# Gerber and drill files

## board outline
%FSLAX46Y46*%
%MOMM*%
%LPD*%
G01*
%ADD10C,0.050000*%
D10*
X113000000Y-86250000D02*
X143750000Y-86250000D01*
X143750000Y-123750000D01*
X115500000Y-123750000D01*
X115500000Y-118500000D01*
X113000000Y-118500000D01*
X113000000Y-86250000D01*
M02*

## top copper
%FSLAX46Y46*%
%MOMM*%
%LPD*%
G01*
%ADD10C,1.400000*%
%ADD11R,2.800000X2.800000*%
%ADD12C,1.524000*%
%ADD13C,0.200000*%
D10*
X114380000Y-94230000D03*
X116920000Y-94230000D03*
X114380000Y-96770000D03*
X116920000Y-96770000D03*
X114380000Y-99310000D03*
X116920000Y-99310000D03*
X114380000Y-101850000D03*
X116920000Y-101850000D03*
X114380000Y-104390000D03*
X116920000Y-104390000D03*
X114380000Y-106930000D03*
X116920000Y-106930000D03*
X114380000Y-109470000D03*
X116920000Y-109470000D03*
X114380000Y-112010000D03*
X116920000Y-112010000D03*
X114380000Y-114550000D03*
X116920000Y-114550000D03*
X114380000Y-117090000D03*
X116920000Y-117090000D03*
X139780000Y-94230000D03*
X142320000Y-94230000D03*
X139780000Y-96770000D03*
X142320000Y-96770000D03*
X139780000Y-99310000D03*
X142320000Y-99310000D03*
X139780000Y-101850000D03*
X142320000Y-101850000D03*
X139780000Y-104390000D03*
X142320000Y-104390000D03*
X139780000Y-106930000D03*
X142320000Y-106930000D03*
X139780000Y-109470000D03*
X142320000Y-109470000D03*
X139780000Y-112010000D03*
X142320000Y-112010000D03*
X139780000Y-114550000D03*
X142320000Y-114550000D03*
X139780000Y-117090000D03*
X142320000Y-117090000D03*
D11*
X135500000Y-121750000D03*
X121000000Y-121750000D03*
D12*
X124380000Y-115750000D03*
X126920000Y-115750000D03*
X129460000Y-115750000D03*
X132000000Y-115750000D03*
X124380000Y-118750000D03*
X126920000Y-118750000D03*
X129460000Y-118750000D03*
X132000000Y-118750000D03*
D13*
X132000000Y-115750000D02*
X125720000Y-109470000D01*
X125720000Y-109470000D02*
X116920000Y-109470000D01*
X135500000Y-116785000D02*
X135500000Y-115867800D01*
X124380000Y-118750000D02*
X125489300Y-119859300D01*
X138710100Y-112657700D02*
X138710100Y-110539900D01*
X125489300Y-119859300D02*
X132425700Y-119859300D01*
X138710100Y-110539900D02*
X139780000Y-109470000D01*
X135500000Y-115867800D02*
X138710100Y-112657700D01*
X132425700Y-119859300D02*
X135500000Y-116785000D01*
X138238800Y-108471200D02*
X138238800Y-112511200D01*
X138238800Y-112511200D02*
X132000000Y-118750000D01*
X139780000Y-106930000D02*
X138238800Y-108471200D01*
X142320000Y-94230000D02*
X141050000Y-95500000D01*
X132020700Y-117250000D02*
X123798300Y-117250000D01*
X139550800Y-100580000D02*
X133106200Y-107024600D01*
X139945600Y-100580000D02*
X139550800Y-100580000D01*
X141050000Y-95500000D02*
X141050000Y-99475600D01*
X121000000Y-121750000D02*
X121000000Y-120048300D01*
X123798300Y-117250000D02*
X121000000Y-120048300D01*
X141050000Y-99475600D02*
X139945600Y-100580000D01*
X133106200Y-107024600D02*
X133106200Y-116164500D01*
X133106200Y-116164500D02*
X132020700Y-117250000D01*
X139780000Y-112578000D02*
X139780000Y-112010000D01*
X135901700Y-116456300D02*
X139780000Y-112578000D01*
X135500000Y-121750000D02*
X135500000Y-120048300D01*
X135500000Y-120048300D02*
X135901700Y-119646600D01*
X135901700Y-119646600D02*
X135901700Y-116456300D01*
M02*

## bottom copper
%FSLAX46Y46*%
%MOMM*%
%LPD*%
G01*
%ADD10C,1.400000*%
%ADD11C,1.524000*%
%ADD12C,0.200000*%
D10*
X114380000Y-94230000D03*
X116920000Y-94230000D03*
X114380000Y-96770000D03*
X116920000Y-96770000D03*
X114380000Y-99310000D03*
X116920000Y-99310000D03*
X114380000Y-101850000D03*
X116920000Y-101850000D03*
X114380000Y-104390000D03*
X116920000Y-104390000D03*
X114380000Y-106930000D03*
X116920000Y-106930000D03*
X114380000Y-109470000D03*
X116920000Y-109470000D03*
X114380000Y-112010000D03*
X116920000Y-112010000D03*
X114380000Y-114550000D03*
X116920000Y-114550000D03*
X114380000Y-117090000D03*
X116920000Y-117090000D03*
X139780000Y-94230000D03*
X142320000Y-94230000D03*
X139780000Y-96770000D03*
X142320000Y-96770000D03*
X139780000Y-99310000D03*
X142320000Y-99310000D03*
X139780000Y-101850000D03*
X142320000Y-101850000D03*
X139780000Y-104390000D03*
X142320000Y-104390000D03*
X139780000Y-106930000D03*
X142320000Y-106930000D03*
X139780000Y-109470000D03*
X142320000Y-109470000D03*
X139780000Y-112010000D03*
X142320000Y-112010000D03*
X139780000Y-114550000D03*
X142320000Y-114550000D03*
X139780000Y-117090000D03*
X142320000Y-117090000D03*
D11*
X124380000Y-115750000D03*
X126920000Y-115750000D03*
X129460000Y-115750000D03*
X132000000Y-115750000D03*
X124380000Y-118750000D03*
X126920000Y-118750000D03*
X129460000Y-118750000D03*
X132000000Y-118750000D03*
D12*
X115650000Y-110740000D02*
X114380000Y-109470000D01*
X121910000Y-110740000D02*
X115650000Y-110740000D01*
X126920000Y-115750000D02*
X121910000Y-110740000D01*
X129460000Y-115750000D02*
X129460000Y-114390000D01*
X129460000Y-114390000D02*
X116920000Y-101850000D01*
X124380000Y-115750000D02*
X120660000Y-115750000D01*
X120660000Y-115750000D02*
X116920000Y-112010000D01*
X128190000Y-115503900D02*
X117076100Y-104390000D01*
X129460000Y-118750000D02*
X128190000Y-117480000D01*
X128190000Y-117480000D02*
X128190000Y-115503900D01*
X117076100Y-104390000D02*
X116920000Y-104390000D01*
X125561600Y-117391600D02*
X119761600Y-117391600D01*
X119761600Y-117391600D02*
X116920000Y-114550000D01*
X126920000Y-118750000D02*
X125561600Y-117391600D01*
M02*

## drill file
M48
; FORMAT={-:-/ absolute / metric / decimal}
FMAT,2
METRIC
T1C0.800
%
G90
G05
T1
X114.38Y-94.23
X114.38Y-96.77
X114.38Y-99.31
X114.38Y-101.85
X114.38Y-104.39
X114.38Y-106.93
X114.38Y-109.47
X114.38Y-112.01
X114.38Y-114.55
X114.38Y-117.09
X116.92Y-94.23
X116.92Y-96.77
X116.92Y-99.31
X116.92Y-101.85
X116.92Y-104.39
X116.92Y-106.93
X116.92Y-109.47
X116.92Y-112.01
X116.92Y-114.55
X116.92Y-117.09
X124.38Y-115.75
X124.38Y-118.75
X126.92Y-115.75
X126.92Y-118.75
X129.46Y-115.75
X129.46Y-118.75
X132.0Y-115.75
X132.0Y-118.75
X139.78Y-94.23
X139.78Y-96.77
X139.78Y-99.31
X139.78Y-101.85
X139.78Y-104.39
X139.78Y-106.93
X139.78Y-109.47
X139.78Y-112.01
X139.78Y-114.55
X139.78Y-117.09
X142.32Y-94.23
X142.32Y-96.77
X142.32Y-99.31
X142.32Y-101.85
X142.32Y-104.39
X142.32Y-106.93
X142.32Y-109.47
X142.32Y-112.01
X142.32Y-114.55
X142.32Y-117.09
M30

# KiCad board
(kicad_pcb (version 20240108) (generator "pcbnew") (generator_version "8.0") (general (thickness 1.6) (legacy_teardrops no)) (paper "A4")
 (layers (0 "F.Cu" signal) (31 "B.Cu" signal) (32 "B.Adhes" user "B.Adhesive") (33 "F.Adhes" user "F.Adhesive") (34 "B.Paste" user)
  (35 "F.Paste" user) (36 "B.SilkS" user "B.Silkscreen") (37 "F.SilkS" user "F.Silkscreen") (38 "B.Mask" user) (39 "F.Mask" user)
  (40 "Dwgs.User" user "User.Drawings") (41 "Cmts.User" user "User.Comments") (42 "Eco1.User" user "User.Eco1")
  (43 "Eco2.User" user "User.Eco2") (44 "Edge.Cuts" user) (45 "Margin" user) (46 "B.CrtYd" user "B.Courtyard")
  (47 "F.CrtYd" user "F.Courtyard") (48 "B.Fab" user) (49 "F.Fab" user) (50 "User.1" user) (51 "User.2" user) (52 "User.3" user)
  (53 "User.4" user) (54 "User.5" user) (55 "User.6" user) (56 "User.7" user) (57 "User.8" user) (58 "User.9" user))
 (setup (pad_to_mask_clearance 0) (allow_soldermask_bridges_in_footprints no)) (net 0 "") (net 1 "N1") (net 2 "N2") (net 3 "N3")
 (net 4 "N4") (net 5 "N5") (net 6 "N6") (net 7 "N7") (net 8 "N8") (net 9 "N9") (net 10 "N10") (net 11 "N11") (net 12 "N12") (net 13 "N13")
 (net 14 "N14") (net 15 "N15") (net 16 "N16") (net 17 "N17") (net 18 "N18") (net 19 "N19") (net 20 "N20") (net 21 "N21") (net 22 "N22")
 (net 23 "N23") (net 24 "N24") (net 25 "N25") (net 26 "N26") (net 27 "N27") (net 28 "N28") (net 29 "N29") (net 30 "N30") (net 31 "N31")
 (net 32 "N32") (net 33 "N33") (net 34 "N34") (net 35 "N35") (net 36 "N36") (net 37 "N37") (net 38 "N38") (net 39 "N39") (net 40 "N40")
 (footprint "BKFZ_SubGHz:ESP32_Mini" (layer "F.Cu") (at 128.35 105.66)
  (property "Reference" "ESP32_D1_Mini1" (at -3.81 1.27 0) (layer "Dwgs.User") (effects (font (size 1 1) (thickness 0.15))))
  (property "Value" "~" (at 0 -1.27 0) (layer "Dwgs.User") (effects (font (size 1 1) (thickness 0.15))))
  (pad "1" thru_hole circle (at -13.97 -11.43 270) (size 1.4 1.4) (drill 0.8) (layers "*.Cu" "*.Mask") (remove_unused_layers no)
   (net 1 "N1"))
  (pad "2" thru_hole circle (at -11.43 -11.43 270) (size 1.4 1.4) (drill 0.8) (layers "*.Cu" "*.Mask") (remove_unused_layers no)
   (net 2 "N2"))
  (pad "3" thru_hole circle (at -13.97 -8.89 270) (size 1.4 1.4) (drill 0.8) (layers "*.Cu" "*.Mask") (remove_unused_layers no) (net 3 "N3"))
  (pad "4" thru_hole circle (at -11.43 -8.89 270) (size 1.4 1.4) (drill 0.8) (layers "*.Cu" "*.Mask") (remove_unused_layers no) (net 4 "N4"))
  (pad "5" thru_hole circle (at -13.97 -6.35 270) (size 1.4 1.4) (drill 0.8) (layers "*.Cu" "*.Mask") (remove_unused_layers no) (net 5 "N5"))
  (pad "6" thru_hole circle (at -11.43 -6.35 270) (size 1.4 1.4) (drill 0.8) (layers "*.Cu" "*.Mask") (remove_unused_layers no) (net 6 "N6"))
  (pad "7" thru_hole circle (at -13.97 -3.81 270) (size 1.4 1.4) (drill 0.8) (layers "*.Cu" "*.Mask") (remove_unused_layers no) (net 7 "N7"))
  (pad "8" thru_hole circle (at -11.43 -3.81 270) (size 1.4 1.4) (drill 0.8) (layers "*.Cu" "*.Mask") (remove_unused_layers no) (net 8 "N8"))
  (pad "9" thru_hole circle (at -13.97 -1.27 270) (size 1.4 1.4) (drill 0.8) (layers "*.Cu" "*.Mask") (remove_unused_layers no) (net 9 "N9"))
  (pad "10" thru_hole circle (at -11.43 -1.27 270) (size 1.4 1.4) (drill 0.8) (layers "*.Cu" "*.Mask") (remove_unused_layers no)
   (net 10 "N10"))
  (pad "11" thru_hole circle (at -13.97 1.27 270) (size 1.4 1.4) (drill 0.8) (layers "*.Cu" "*.Mask") (remove_unused_layers no)
   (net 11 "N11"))
  (pad "12" thru_hole circle (at -11.43 1.27 270) (size 1.4 1.4) (drill 0.8) (layers "*.Cu" "*.Mask") (remove_unused_layers no)
   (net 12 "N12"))
  (pad "13" thru_hole circle (at -13.97 3.81 270) (size 1.4 1.4) (drill 0.8) (layers "*.Cu" "*.Mask") (remove_unused_layers no)
   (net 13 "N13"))
  (pad "14" thru_hole circle (at -11.43 3.81 270) (size 1.4 1.4) (drill 0.8) (layers "*.Cu" "*.Mask") (remove_unused_layers no)
   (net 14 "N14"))
  (pad "15" thru_hole circle (at -13.97 6.35 270) (size 1.4 1.4) (drill 0.8) (layers "*.Cu" "*.Mask") (remove_unused_layers no)
   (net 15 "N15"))
  (pad "16" thru_hole circle (at -11.43 6.35 270) (size 1.4 1.4) (drill 0.8) (layers "*.Cu" "*.Mask") (remove_unused_layers no)
   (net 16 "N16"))
  (pad "17" thru_hole circle (at -13.97 8.89 270) (size 1.4 1.4) (drill 0.8) (layers "*.Cu" "*.Mask") (remove_unused_layers no)
   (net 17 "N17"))
  (pad "18" thru_hole circle (at -11.43 8.89 270) (size 1.4 1.4) (drill 0.8) (layers "*.Cu" "*.Mask") (remove_unused_layers no)
   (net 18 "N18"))
  (pad "19" thru_hole circle (at -13.97 11.43 270) (size 1.4 1.4) (drill 0.8) (layers "*.Cu" "*.Mask") (remove_unused_layers no)
   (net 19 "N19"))
  (pad "20" thru_hole circle (at -11.43 11.43 270) (size 1.4 1.4) (drill 0.8) (layers "*.Cu" "*.Mask") (remove_unused_layers no)
   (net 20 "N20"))
  (pad "21" thru_hole circle (at 11.43 -11.43 270) (size 1.4 1.4) (drill 0.8) (layers "*.Cu" "*.Mask") (remove_unused_layers no)
   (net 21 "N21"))
  (pad "22" thru_hole circle (at 13.97 -11.43 270) (size 1.4 1.4) (drill 0.8) (layers "*.Cu" "*.Mask") (remove_unused_layers no)
   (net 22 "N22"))
  (pad "23" thru_hole circle (at 11.43 -8.89 270) (size 1.4 1.4) (drill 0.8) (layers "*.Cu" "*.Mask") (remove_unused_layers no)
   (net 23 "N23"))
  (pad "24" thru_hole circle (at 13.97 -8.89 270) (size 1.4 1.4) (drill 0.8) (layers "*.Cu" "*.Mask") (remove_unused_layers no)
   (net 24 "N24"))
  (pad "25" thru_hole circle (at 11.43 -6.35 270) (size 1.4 1.4) (drill 0.8) (layers "*.Cu" "*.Mask") (remove_unused_layers no)
   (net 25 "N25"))
  (pad "26" thru_hole circle (at 13.97 -6.35 270) (size 1.4 1.4) (drill 0.8) (layers "*.Cu" "*.Mask") (remove_unused_layers no)
   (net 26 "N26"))
  (pad "27" thru_hole circle (at 11.43 -3.81 270) (size 1.4 1.4) (drill 0.8) (layers "*.Cu" "*.Mask") (remove_unused_layers no)
   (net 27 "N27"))
  (pad "28" thru_hole circle (at 13.97 -3.81 270) (size 1.4 1.4) (drill 0.8) (layers "*.Cu" "*.Mask") (remove_unused_layers no)
   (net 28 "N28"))
  (pad "29" thru_hole circle (at 11.43 -1.27 270) (size 1.4 1.4) (drill 0.8) (layers "*.Cu" "*.Mask") (remove_unused_layers no)
   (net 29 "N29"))
  (pad "30" thru_hole circle (at 13.97 -1.27 270) (size 1.4 1.4) (drill 0.8) (layers "*.Cu" "*.Mask") (remove_unused_layers no)
   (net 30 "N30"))
  (pad "31" thru_hole circle (at 11.43 1.27 270) (size 1.4 1.4) (drill 0.8) (layers "*.Cu" "*.Mask") (remove_unused_layers no)
   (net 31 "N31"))
  (pad "32" thru_hole circle (at 13.97 1.27 270) (size 1.4 1.4) (drill 0.8) (layers "*.Cu" "*.Mask") (remove_unused_layers no)
   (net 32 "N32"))
  (pad "33" thru_hole circle (at 11.43 3.81 270) (size 1.4 1.4) (drill 0.8) (layers "*.Cu" "*.Mask") (remove_unused_layers no)
   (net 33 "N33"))
  (pad "34" thru_hole circle (at 13.97 3.81 270) (size 1.4 1.4) (drill 0.8) (layers "*.Cu" "*.Mask") (remove_unused_layers no)
   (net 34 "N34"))
  (pad "35" thru_hole circle (at 11.43 6.35 270) (size 1.4 1.4) (drill 0.8) (layers "*.Cu" "*.Mask") (remove_unused_layers no)
   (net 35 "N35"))
  (pad "36" thru_hole circle (at 13.97 6.35 270) (size 1.4 1.4) (drill 0.8) (layers "*.Cu" "*.Mask") (remove_unused_layers no)
   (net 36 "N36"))
  (pad "37" thru_hole circle (at 11.43 8.89 270) (size 1.4 1.4) (drill 0.8) (layers "*.Cu" "*.Mask") (remove_unused_layers no)
   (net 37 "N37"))
  (pad "38" thru_hole circle (at 13.97 8.89 270) (size 1.4 1.4) (drill 0.8) (layers "*.Cu" "*.Mask") (remove_unused_layers no)
   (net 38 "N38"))
  (pad "39" thru_hole circle (at 11.43 11.43 270) (size 1.4 1.4) (drill 0.8) (layers "*.Cu" "*.Mask") (remove_unused_layers no)
   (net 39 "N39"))
  (pad "40" thru_hole circle (at 13.97 11.43 270) (size 1.4 1.4) (drill 0.8) (layers "*.Cu" "*.Mask") (remove_unused_layers no)
   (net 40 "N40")))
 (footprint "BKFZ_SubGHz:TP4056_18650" (layer "F.Cu") (at 137.2 97.15 -90)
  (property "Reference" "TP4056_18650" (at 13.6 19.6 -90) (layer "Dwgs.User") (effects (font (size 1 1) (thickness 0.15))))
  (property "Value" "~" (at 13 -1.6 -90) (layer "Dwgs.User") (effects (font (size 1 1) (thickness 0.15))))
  (pad "3" smd rect (at 24.6 1.7 270) (size 2.8 2.8) (layers "F.Cu" "F.Paste" "F.Mask") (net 35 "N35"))
  (pad "4" smd rect (at 24.6 16.2 270) (size 2.8 2.8) (layers "F.Cu" "F.Paste" "F.Mask") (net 22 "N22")))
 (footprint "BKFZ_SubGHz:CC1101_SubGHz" (layer "F.Cu") (at 153.685 71.9)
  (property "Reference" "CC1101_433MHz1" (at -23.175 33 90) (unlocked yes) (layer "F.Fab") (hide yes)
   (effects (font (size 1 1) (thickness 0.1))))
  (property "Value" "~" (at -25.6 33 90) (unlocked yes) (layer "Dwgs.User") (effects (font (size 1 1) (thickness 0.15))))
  (pad "1" thru_hole circle (at -29.305 43.85 270) (size 1.524 1.524) (drill 0.8) (layers "*.Cu" "*.Mask") (remove_unused_layers no)
   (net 16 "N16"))
  (pad "2" thru_hole circle (at -26.765 43.85 270) (size 1.524 1.524) (drill 0.8) (layers "*.Cu" "*.Mask") (remove_unused_layers no)
   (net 13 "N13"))
  (pad "3" thru_hole circle (at -24.225 43.85 270) (size 1.524 1.524) (drill 0.8) (layers "*.Cu" "*.Mask") (remove_unused_layers no)
   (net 8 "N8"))
  (pad "4" thru_hole circle (at -21.685 43.85 270) (size 1.524 1.524) (drill 0.8) (layers "*.Cu" "*.Mask") (remove_unused_layers no)
   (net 14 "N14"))
  (pad "5" thru_hole circle (at -29.305 46.85 270) (size 1.524 1.524) (drill 0.8) (layers "*.Cu" "*.Mask") (remove_unused_layers no)
   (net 33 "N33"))
  (pad "6" thru_hole circle (at -26.765 46.85 270) (size 1.524 1.524) (drill 0.8) (layers "*.Cu" "*.Mask") (remove_unused_layers no)
   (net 18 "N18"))
  (pad "7" thru_hole circle (at -24.225 46.85 270) (size 1.524 1.524) (drill 0.8) (layers "*.Cu" "*.Mask") (remove_unused_layers no)
   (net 10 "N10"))
  (pad "8" thru_hole circle (at -21.685 46.85 270) (size 1.524 1.524) (drill 0.8) (layers "*.Cu" "*.Mask") (remove_unused_layers no)
   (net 31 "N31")))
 (gr_poly
  (pts (xy 113 86.25) (xy 143.75 86.25) (xy 143.75 123.75) (xy 115.5 123.75) (xy 115.5 118.5) (xy 113 118.5))
  (stroke (width 0.05) (type solid)) (fill none) (layer "Edge.Cuts"))
 (segment (start 115.65 110.74) (end 114.38 109.47) (width 0.2) (layer "B.Cu") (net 13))
 (segment (start 121.91 110.74) (end 115.65 110.74) (width 0.2) (layer "B.Cu") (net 13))
 (segment (start 126.92 115.75) (end 121.91 110.74) (width 0.2) (layer "B.Cu") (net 13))
 (segment (start 129.46 115.75) (end 129.46 114.39) (width 0.2) (layer "B.Cu") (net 8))
 (segment (start 129.46 114.39) (end 116.92 101.85) (width 0.2) (layer "B.Cu") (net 8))
 (segment (start 132 115.75) (end 125.72 109.47) (width 0.2) (layer "F.Cu") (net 14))
 (segment (start 125.72 109.47) (end 116.92 109.47) (width 0.2) (layer "F.Cu") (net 14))
 (segment (start 124.38 115.75) (end 120.66 115.75) (width 0.2) (layer "B.Cu") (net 16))
 (segment (start 120.66 115.75) (end 116.92 112.01) (width 0.2) (layer "B.Cu") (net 16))
 (segment (start 135.5 116.785) (end 135.5 115.8678) (width 0.2) (layer "F.Cu") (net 33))
 (segment (start 124.38 118.75) (end 125.4893 119.8593) (width 0.2) (layer "F.Cu") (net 33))
 (segment (start 138.7101 112.6577) (end 138.7101 110.5399) (width 0.2) (layer "F.Cu") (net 33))
 (segment (start 125.4893 119.8593) (end 132.4257 119.8593) (width 0.2) (layer "F.Cu") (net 33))
 (segment (start 138.7101 110.5399) (end 139.78 109.47) (width 0.2) (layer "F.Cu") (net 33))
 (segment (start 135.5 115.8678) (end 138.7101 112.6577) (width 0.2) (layer "F.Cu") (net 33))
 (segment (start 132.4257 119.8593) (end 135.5 116.785) (width 0.2) (layer "F.Cu") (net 33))
 (segment (start 128.19 115.5039) (end 117.0761 104.39) (width 0.2) (layer "B.Cu") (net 10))
 (segment (start 129.46 118.75) (end 128.19 117.48) (width 0.2) (layer "B.Cu") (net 10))
 (segment (start 128.19 117.48) (end 128.19 115.5039) (width 0.2) (layer "B.Cu") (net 10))
 (segment (start 117.0761 104.39) (end 116.92 104.39) (width 0.2) (layer "B.Cu") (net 10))
 (segment (start 138.2388 108.4712) (end 138.2388 112.5112) (width 0.2) (layer "F.Cu") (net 31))
 (segment (start 138.2388 112.5112) (end 132 118.75) (width 0.2) (layer "F.Cu") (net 31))
 (segment (start 139.78 106.93) (end 138.2388 108.4712) (width 0.2) (layer "F.Cu") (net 31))
 (segment (start 125.5616 117.3916) (end 119.7616 117.3916) (width 0.2) (layer "B.Cu") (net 18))
 (segment (start 119.7616 117.3916) (end 116.92 114.55) (width 0.2) (layer "B.Cu") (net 18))
 (segment (start 126.92 118.75) (end 125.5616 117.3916) (width 0.2) (layer "B.Cu") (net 18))
 (segment (start 142.32 94.23) (end 141.05 95.5) (width 0.2) (layer "F.Cu") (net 22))
 (segment (start 132.0207 117.25) (end 123.7983 117.25) (width 0.2) (layer "F.Cu") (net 22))
 (segment (start 139.5508 100.58) (end 133.1062 107.0246) (width 0.2) (layer "F.Cu") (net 22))
 (segment (start 139.9456 100.58) (end 139.5508 100.58) (width 0.2) (layer "F.Cu") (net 22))
 (segment (start 141.05 95.5) (end 141.05 99.4756) (width 0.2) (layer "F.Cu") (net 22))
 (segment (start 121 121.75) (end 121 120.0483) (width 0.2) (layer "F.Cu") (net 22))
 (segment (start 123.7983 117.25) (end 121 120.0483) (width 0.2) (layer "F.Cu") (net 22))
 (segment (start 141.05 99.4756) (end 139.9456 100.58) (width 0.2) (layer "F.Cu") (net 22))
 (segment (start 133.1062 107.0246) (end 133.1062 116.1645) (width 0.2) (layer "F.Cu") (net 22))
 (segment (start 133.1062 116.1645) (end 132.0207 117.25) (width 0.2) (layer "F.Cu") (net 22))
 (segment (start 139.78 112.578) (end 139.78 112.01) (width 0.2) (layer "F.Cu") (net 35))
 (segment (start 135.9017 116.4563) (end 139.78 112.578) (width 0.2) (layer "F.Cu") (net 35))
 (segment (start 135.5 121.75) (end 135.5 120.0483) (width 0.2) (layer "F.Cu") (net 35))
 (segment (start 135.5 120.0483) (end 135.9017 119.6466) (width 0.2) (layer "F.Cu") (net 35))
 (segment (start 135.9017 119.6466) (end 135.9017 116.4563) (width 0.2) (layer "F.Cu") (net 35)))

